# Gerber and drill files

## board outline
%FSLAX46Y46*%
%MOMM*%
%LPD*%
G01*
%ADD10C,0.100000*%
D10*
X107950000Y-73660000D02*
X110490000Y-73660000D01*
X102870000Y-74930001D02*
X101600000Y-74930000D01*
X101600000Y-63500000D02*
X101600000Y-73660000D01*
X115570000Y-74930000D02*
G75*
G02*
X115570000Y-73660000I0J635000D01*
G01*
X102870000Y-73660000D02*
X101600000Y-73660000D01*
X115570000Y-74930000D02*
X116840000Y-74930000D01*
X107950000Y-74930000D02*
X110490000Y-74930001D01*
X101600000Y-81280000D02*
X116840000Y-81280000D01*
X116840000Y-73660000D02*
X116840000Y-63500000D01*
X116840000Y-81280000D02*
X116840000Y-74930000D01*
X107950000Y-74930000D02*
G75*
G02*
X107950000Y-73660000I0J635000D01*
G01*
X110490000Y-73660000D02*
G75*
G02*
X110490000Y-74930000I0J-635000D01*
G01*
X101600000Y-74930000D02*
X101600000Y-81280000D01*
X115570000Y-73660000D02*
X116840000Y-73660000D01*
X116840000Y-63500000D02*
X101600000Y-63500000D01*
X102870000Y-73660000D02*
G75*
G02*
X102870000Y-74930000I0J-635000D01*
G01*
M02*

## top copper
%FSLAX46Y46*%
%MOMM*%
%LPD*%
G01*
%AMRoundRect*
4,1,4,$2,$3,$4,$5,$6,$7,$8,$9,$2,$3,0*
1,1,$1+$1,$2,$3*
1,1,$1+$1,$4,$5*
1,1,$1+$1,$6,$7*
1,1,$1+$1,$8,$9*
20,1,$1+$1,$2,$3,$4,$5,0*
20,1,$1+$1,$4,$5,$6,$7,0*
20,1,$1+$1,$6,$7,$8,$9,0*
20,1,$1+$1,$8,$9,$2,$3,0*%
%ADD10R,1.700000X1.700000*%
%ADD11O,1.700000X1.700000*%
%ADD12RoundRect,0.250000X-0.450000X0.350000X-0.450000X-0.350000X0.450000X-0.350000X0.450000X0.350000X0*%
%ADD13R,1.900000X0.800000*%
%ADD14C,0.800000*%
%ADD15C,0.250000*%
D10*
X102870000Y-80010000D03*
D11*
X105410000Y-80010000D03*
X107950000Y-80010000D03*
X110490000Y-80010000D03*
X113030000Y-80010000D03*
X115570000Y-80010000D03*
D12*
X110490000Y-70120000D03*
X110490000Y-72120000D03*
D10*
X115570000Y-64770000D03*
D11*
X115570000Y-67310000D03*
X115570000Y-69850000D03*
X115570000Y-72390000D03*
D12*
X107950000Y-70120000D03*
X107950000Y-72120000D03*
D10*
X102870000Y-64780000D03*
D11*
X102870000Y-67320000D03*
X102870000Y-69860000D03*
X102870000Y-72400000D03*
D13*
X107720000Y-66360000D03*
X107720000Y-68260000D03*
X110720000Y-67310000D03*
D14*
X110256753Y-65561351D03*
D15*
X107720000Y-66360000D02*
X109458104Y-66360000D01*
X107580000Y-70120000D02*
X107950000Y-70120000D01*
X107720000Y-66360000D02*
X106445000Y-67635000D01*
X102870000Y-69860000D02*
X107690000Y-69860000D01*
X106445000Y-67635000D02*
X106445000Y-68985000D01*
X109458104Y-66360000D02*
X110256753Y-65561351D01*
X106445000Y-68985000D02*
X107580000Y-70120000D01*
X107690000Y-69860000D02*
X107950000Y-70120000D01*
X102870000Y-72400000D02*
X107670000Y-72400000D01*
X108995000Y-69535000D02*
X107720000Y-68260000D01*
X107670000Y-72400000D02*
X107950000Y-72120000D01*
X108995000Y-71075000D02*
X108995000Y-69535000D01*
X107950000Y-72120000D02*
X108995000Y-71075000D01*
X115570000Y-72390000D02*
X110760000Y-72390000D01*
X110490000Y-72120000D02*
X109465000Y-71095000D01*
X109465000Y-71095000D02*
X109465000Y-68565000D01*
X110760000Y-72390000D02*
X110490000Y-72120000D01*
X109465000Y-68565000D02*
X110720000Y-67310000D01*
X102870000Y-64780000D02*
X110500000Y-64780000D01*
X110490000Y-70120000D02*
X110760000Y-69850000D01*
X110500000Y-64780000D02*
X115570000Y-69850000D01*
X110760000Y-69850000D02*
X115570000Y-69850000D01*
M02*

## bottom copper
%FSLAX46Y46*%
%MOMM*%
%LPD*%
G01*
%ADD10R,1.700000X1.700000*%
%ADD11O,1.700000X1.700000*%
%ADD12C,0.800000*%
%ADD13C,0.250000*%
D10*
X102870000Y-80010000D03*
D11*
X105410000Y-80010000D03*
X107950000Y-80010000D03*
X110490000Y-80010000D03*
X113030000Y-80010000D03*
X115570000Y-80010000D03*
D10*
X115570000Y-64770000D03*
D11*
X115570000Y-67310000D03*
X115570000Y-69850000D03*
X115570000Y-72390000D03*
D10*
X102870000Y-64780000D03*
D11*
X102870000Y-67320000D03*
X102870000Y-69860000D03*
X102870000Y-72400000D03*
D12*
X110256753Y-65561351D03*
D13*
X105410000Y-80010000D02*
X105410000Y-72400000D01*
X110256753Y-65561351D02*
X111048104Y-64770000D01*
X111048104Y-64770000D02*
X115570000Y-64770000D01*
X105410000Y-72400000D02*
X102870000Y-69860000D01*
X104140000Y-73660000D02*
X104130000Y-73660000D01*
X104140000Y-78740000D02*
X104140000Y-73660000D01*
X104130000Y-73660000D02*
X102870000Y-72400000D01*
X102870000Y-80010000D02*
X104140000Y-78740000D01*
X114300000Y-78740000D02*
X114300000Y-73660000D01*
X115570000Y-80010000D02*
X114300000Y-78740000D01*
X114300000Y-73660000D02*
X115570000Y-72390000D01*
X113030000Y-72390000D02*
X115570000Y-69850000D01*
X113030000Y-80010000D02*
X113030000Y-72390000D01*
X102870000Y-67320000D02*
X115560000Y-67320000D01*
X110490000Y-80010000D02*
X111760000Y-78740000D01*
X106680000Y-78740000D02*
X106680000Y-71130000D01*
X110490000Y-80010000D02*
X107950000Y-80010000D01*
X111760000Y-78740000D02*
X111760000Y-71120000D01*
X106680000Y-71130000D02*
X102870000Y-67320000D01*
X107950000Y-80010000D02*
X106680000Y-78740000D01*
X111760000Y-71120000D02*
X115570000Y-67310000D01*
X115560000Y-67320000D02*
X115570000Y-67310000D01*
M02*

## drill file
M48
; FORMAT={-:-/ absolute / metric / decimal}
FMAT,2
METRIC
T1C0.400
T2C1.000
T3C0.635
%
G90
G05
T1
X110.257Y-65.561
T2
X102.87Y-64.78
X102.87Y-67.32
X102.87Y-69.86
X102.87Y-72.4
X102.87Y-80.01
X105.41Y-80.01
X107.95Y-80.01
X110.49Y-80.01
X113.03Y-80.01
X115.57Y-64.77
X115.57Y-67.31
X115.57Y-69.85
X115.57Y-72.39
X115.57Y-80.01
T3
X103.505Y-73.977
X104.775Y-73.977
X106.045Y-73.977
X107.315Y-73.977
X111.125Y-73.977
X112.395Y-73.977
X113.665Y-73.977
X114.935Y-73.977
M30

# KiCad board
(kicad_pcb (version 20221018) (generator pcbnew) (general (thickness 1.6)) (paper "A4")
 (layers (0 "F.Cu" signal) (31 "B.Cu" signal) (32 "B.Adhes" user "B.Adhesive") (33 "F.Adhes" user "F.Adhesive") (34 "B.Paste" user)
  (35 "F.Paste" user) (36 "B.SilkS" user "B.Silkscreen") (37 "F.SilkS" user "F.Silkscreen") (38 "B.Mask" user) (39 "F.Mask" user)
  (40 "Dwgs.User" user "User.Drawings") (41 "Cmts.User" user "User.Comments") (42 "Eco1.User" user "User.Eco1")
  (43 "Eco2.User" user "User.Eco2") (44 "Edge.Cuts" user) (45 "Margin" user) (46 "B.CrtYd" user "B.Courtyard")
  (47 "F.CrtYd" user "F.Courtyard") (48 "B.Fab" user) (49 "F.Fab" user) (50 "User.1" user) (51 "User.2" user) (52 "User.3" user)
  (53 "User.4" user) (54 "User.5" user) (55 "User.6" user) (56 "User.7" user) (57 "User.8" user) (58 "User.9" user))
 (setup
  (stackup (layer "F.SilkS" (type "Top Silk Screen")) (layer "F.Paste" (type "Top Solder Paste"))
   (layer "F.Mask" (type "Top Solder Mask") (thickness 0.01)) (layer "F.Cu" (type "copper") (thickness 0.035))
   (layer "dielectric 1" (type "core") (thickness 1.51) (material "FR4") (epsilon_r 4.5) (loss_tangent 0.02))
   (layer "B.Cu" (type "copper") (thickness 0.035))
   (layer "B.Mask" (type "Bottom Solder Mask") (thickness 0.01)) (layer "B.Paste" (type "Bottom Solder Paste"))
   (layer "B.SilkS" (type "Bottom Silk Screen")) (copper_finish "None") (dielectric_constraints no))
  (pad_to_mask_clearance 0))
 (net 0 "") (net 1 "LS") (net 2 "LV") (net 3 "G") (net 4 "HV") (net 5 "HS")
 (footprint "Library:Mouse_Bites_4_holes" (layer "F.Cu") (at 105.41 73.66 180)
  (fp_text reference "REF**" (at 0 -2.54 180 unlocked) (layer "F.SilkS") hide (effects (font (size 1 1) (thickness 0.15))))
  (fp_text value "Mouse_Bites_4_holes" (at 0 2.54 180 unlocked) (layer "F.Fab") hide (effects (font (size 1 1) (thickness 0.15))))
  (pad "" np_thru_hole circle (at -1.905 -0.3175 180) (size 0.635 0.635) (drill 0.635) (layers "*.Mask") (thermal_bridge_angle 90))
  (pad "" np_thru_hole circle (at -0.635 -0.3175 180) (size 0.635 0.635) (drill 0.635) (layers "*.Mask") (thermal_bridge_angle 90))
  (pad "" np_thru_hole circle (at 0.635 -0.3175 180) (size 0.635 0.635) (drill 0.635) (layers "*.Mask") (thermal_bridge_angle 90))
  (pad "" np_thru_hole circle (at 1.905 -0.3175 180) (size 0.635 0.635) (drill 0.635) (layers "*.Mask") (thermal_bridge_angle 90)))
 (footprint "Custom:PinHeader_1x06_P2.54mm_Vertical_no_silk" (layer "F.Cu") (at 102.87 80.01 90)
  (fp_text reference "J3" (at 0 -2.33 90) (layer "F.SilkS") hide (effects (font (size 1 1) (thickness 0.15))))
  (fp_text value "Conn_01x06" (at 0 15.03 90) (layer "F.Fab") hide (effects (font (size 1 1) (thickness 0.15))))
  (pad "1" thru_hole rect (at 0 0 90) (size 1.7 1.7) (drill 1) (layers "*.Cu" "*.Mask") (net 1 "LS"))
  (pad "2" thru_hole oval (at 0 2.54 90) (size 1.7 1.7) (drill 1) (layers "*.Cu" "*.Mask") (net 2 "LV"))
  (pad "3" thru_hole oval (at 0 5.08 90) (size 1.7 1.7) (drill 1) (layers "*.Cu" "*.Mask") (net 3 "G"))
  (pad "4" thru_hole oval (at 0 7.62 90) (size 1.7 1.7) (drill 1) (layers "*.Cu" "*.Mask") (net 3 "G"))
  (pad "5" thru_hole oval (at 0 10.16 90) (size 1.7 1.7) (drill 1) (layers "*.Cu" "*.Mask") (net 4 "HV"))
  (pad "6" thru_hole oval (at 0 12.7 90) (size 1.7 1.7) (drill 1) (layers "*.Cu" "*.Mask") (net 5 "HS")))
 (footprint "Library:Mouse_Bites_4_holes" (layer "F.Cu") (at 113.03 73.66 180)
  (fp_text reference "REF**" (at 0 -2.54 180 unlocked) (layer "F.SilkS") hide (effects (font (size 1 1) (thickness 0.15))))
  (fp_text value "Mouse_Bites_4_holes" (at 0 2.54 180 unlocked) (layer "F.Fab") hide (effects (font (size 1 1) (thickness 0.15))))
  (pad "" np_thru_hole circle (at -1.905 -0.3175 180) (size 0.635 0.635) (drill 0.635) (layers "*.Mask") (thermal_bridge_angle 90))
  (pad "" np_thru_hole circle (at -0.635 -0.3175 180) (size 0.635 0.635) (drill 0.635) (layers "*.Mask") (thermal_bridge_angle 90))
  (pad "" np_thru_hole circle (at 0.635 -0.3175 180) (size 0.635 0.635) (drill 0.635) (layers "*.Mask") (thermal_bridge_angle 90))
  (pad "" np_thru_hole circle (at 1.905 -0.3175 180) (size 0.635 0.635) (drill 0.635) (layers "*.Mask") (thermal_bridge_angle 90)))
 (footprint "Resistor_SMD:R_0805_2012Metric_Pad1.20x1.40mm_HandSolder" (layer "F.Cu") (at 110.49 71.12 -90)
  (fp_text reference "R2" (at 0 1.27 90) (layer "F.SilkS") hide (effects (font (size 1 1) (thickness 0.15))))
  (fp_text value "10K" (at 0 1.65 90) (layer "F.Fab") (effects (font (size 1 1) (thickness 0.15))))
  (pad "1" smd roundrect (at -1 0 270) (size 1.2 1.4) (layers "F.Cu" "F.Paste" "F.Mask") (roundrect_rratio 0.208333) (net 4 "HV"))
  (pad "2" smd roundrect (at 1 0 270) (size 1.2 1.4) (layers "F.Cu" "F.Paste" "F.Mask") (roundrect_rratio 0.208333) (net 5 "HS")))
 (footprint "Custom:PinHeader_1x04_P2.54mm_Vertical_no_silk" (layer "F.Cu") (at 115.57 64.77)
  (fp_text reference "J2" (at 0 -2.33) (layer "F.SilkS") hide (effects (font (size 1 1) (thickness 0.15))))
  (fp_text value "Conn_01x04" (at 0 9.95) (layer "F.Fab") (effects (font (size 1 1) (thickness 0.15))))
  (pad "1" thru_hole rect (at 0 0) (size 1.7 1.7) (drill 1) (layers "*.Cu" "*.Mask") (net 2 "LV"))
  (pad "2" thru_hole oval (at 0 2.54) (size 1.7 1.7) (drill 1) (layers "*.Cu" "*.Mask") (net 3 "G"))
  (pad "3" thru_hole oval (at 0 5.08) (size 1.7 1.7) (drill 1) (layers "*.Cu" "*.Mask") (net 4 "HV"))
  (pad "4" thru_hole oval (at 0 7.62) (size 1.7 1.7) (drill 1) (layers "*.Cu" "*.Mask") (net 5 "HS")))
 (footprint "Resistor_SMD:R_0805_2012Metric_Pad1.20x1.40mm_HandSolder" (layer "F.Cu") (at 107.95 71.12 -90)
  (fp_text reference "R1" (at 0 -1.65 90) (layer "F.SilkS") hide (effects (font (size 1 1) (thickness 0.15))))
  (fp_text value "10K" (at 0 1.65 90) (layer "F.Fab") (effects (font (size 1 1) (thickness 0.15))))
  (pad "1" smd roundrect (at -1 0 270) (size 1.2 1.4) (layers "F.Cu" "F.Paste" "F.Mask") (roundrect_rratio 0.208333) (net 2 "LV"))
  (pad "2" smd roundrect (at 1 0 270) (size 1.2 1.4) (layers "F.Cu" "F.Paste" "F.Mask") (roundrect_rratio 0.208333) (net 1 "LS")))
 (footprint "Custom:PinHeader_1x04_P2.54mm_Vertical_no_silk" (layer "F.Cu") (at 102.87 64.78)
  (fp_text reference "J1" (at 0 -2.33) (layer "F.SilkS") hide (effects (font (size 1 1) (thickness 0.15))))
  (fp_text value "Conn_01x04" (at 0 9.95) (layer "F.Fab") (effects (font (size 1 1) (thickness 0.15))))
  (pad "1" thru_hole rect (at 0 0) (size 1.7 1.7) (drill 1) (layers "*.Cu" "*.Mask") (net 4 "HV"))
  (pad "2" thru_hole oval (at 0 2.54) (size 1.7 1.7) (drill 1) (layers "*.Cu" "*.Mask") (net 3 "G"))
  (pad "3" thru_hole oval (at 0 5.08) (size 1.7 1.7) (drill 1) (layers "*.Cu" "*.Mask") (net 2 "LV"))
  (pad "4" thru_hole oval (at 0 7.62) (size 1.7 1.7) (drill 1) (layers "*.Cu" "*.Mask") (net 1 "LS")))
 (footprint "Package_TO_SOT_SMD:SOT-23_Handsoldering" (layer "F.Cu") (at 109.22 67.31)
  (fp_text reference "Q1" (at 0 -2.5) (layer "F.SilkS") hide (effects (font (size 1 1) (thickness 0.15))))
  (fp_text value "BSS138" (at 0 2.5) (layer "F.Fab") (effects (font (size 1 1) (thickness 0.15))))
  (pad "1" smd rect (at -1.5 -0.95) (size 1.9 0.8) (layers "F.Cu" "F.Paste" "F.Mask") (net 2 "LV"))
  (pad "2" smd rect (at -1.5 0.95) (size 1.9 0.8) (layers "F.Cu" "F.Paste" "F.Mask") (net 1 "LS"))
  (pad "3" smd rect (at 1.5 0) (size 1.9 0.8) (layers "F.Cu" "F.Paste" "F.Mask") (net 5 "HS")))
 (gr_line (start 107.95 73.66) (end 110.49 73.66) (stroke (width 0.1) (type default)) (layer "Edge.Cuts"))
 (gr_line (start 102.87 74.930001) (end 101.6 74.93) (stroke (width 0.1) (type default)) (layer "Edge.Cuts"))
 (gr_line (start 101.6 63.5) (end 101.6 73.66) (stroke (width 0.1) (type default)) (layer "Edge.Cuts"))
 (gr_arc (start 115.57 74.93) (mid 114.935 74.295) (end 115.57 73.66) (stroke (width 0.1) (type default)) (layer "Edge.Cuts"))
 (gr_line (start 102.87 73.66) (end 101.6 73.66) (stroke (width 0.1) (type default)) (layer "Edge.Cuts"))
 (gr_line (start 115.57 74.93) (end 116.84 74.93) (stroke (width 0.1) (type default)) (layer "Edge.Cuts"))
 (gr_line (start 107.95 74.93) (end 110.49 74.930001) (stroke (width 0.1) (type default)) (layer "Edge.Cuts"))
 (gr_line (start 101.6 81.28) (end 116.84 81.28) (stroke (width 0.1) (type default)) (layer "Edge.Cuts"))
 (gr_line (start 116.84 73.66) (end 116.84 63.5) (stroke (width 0.1) (type default)) (layer "Edge.Cuts"))
 (gr_line (start 116.84 81.28) (end 116.84 74.93) (stroke (width 0.1) (type default)) (layer "Edge.Cuts"))
 (gr_arc (start 107.95 74.93) (mid 107.315 74.295) (end 107.95 73.66) (stroke (width 0.1) (type default)) (layer "Edge.Cuts"))
 (gr_arc (start 110.49 73.66) (mid 111.125 74.295) (end 110.49 74.930001) (stroke (width 0.1) (type default)) (layer "Edge.Cuts"))
 (gr_line (start 101.6 74.93) (end 101.6 81.28) (stroke (width 0.1) (type default)) (layer "Edge.Cuts"))
 (gr_line (start 115.57 73.66) (end 116.84 73.66) (stroke (width 0.1) (type default)) (layer "Edge.Cuts"))
 (gr_line (start 116.84 63.5) (end 101.6 63.5) (stroke (width 0.1) (type default)) (layer "Edge.Cuts"))
 (gr_arc (start 102.87 73.66) (mid 103.505 74.295) (end 102.87 74.930001) (stroke (width 0.1) (type default)) (layer "Edge.Cuts"))
 (segment (start 107.72 66.36) (end 109.458104 66.36) (width 0.25) (layer "F.Cu") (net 2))
 (segment (start 107.58 70.12) (end 107.95 70.12) (width 0.25) (layer "F.Cu") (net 2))
 (segment (start 107.72 66.36) (end 106.445 67.635) (width 0.25) (layer "F.Cu") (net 2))
 (segment (start 102.87 69.86) (end 107.69 69.86) (width 0.25) (layer "F.Cu") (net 2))
 (segment (start 106.445 67.635) (end 106.445 68.985) (width 0.25) (layer "F.Cu") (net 2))
 (segment (start 109.458104 66.36) (end 110.256753 65.561351) (width 0.25) (layer "F.Cu") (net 2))
 (segment (start 106.445 68.985) (end 107.58 70.12) (width 0.25) (layer "F.Cu") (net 2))
 (segment (start 107.69 69.86) (end 107.95 70.12) (width 0.25) (layer "F.Cu") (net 2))
 (via (at 110.256753 65.561351) (size 0.8) (drill 0.4) (layers "F.Cu" "B.Cu") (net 2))
 (segment (start 105.41 80.01) (end 105.41 72.4) (width 0.25) (layer "B.Cu") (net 2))
 (segment (start 110.256753 65.561351) (end 111.048104 64.77) (width 0.25) (layer "B.Cu") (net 2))
 (segment (start 111.048104 64.77) (end 115.57 64.77) (width 0.25) (layer "B.Cu") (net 2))
 (segment (start 105.41 72.4) (end 102.87 69.86) (width 0.25) (layer "B.Cu") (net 2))
 (segment (start 102.87 72.4) (end 107.67 72.4) (width 0.25) (layer "F.Cu") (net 1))
 (segment (start 108.995 69.535) (end 107.72 68.26) (width 0.25) (layer "F.Cu") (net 1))
 (segment (start 107.67 72.4) (end 107.95 72.12) (width 0.25) (layer "F.Cu") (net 1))
 (segment (start 108.995 71.075) (end 108.995 69.535) (width 0.25) (layer "F.Cu") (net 1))
 (segment (start 107.95 72.12) (end 108.995 71.075) (width 0.25) (layer "F.Cu") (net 1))
 (segment (start 104.14 73.66) (end 104.13 73.66) (width 0.25) (layer "B.Cu") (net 1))
 (segment (start 104.14 78.74) (end 104.14 73.66) (width 0.25) (layer "B.Cu") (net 1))
 (segment (start 104.13 73.66) (end 102.87 72.4) (width 0.25) (layer "B.Cu") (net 1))
 (segment (start 102.87 80.01) (end 104.14 78.74) (width 0.25) (layer "B.Cu") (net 1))
 (segment (start 115.57 72.39) (end 110.76 72.39) (width 0.25) (layer "F.Cu") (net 5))
 (segment (start 110.49 72.12) (end 109.465 71.095) (width 0.25) (layer "F.Cu") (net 5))
 (segment (start 109.465 71.095) (end 109.465 68.565) (width 0.25) (layer "F.Cu") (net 5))
 (segment (start 110.76 72.39) (end 110.49 72.12) (width 0.25) (layer "F.Cu") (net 5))
 (segment (start 109.465 68.565) (end 110.72 67.31) (width 0.25) (layer "F.Cu") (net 5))
 (segment (start 114.3 78.74) (end 114.3 73.66) (width 0.25) (layer "B.Cu") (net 5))
 (segment (start 115.57 80.01) (end 114.3 78.74) (width 0.25) (layer "B.Cu") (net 5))
 (segment (start 114.3 73.66) (end 115.57 72.39) (width 0.25) (layer "B.Cu") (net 5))
 (segment (start 102.87 64.78) (end 110.5 64.78) (width 0.25) (layer "F.Cu") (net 4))
 (segment (start 110.49 70.12) (end 110.76 69.85) (width 0.25) (layer "F.Cu") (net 4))
 (segment (start 110.5 64.78) (end 115.57 69.85) (width 0.25) (layer "F.Cu") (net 4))
 (segment (start 110.76 69.85) (end 115.57 69.85) (width 0.25) (layer "F.Cu") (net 4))
 (segment (start 113.03 72.39) (end 115.57 69.85) (width 0.25) (layer "B.Cu") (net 4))
 (segment (start 113.03 80.01) (end 113.03 72.39) (width 0.25) (layer "B.Cu") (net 4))
 (segment (start 102.87 67.32) (end 115.56 67.32) (width 0.25) (layer "B.Cu") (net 3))
 (segment (start 110.49 80.01) (end 111.76 78.74) (width 0.25) (layer "B.Cu") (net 3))
 (segment (start 106.68 78.74) (end 106.68 71.13) (width 0.25) (layer "B.Cu") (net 3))
 (segment (start 110.49 80.01) (end 107.95 80.01) (width 0.25) (layer "B.Cu") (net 3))
 (segment (start 111.76 78.74) (end 111.76 71.12) (width 0.25) (layer "B.Cu") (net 3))
 (segment (start 106.68 71.13) (end 102.87 67.32) (width 0.25) (layer "B.Cu") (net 3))
 (segment (start 107.95 80.01) (end 106.68 78.74) (width 0.25) (layer "B.Cu") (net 3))
 (segment (start 111.76 71.12) (end 115.57 67.31) (width 0.25) (layer "B.Cu") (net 3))
 (segment (start 115.56 67.32) (end 115.57 67.31) (width 0.25) (layer "B.Cu") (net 3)))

